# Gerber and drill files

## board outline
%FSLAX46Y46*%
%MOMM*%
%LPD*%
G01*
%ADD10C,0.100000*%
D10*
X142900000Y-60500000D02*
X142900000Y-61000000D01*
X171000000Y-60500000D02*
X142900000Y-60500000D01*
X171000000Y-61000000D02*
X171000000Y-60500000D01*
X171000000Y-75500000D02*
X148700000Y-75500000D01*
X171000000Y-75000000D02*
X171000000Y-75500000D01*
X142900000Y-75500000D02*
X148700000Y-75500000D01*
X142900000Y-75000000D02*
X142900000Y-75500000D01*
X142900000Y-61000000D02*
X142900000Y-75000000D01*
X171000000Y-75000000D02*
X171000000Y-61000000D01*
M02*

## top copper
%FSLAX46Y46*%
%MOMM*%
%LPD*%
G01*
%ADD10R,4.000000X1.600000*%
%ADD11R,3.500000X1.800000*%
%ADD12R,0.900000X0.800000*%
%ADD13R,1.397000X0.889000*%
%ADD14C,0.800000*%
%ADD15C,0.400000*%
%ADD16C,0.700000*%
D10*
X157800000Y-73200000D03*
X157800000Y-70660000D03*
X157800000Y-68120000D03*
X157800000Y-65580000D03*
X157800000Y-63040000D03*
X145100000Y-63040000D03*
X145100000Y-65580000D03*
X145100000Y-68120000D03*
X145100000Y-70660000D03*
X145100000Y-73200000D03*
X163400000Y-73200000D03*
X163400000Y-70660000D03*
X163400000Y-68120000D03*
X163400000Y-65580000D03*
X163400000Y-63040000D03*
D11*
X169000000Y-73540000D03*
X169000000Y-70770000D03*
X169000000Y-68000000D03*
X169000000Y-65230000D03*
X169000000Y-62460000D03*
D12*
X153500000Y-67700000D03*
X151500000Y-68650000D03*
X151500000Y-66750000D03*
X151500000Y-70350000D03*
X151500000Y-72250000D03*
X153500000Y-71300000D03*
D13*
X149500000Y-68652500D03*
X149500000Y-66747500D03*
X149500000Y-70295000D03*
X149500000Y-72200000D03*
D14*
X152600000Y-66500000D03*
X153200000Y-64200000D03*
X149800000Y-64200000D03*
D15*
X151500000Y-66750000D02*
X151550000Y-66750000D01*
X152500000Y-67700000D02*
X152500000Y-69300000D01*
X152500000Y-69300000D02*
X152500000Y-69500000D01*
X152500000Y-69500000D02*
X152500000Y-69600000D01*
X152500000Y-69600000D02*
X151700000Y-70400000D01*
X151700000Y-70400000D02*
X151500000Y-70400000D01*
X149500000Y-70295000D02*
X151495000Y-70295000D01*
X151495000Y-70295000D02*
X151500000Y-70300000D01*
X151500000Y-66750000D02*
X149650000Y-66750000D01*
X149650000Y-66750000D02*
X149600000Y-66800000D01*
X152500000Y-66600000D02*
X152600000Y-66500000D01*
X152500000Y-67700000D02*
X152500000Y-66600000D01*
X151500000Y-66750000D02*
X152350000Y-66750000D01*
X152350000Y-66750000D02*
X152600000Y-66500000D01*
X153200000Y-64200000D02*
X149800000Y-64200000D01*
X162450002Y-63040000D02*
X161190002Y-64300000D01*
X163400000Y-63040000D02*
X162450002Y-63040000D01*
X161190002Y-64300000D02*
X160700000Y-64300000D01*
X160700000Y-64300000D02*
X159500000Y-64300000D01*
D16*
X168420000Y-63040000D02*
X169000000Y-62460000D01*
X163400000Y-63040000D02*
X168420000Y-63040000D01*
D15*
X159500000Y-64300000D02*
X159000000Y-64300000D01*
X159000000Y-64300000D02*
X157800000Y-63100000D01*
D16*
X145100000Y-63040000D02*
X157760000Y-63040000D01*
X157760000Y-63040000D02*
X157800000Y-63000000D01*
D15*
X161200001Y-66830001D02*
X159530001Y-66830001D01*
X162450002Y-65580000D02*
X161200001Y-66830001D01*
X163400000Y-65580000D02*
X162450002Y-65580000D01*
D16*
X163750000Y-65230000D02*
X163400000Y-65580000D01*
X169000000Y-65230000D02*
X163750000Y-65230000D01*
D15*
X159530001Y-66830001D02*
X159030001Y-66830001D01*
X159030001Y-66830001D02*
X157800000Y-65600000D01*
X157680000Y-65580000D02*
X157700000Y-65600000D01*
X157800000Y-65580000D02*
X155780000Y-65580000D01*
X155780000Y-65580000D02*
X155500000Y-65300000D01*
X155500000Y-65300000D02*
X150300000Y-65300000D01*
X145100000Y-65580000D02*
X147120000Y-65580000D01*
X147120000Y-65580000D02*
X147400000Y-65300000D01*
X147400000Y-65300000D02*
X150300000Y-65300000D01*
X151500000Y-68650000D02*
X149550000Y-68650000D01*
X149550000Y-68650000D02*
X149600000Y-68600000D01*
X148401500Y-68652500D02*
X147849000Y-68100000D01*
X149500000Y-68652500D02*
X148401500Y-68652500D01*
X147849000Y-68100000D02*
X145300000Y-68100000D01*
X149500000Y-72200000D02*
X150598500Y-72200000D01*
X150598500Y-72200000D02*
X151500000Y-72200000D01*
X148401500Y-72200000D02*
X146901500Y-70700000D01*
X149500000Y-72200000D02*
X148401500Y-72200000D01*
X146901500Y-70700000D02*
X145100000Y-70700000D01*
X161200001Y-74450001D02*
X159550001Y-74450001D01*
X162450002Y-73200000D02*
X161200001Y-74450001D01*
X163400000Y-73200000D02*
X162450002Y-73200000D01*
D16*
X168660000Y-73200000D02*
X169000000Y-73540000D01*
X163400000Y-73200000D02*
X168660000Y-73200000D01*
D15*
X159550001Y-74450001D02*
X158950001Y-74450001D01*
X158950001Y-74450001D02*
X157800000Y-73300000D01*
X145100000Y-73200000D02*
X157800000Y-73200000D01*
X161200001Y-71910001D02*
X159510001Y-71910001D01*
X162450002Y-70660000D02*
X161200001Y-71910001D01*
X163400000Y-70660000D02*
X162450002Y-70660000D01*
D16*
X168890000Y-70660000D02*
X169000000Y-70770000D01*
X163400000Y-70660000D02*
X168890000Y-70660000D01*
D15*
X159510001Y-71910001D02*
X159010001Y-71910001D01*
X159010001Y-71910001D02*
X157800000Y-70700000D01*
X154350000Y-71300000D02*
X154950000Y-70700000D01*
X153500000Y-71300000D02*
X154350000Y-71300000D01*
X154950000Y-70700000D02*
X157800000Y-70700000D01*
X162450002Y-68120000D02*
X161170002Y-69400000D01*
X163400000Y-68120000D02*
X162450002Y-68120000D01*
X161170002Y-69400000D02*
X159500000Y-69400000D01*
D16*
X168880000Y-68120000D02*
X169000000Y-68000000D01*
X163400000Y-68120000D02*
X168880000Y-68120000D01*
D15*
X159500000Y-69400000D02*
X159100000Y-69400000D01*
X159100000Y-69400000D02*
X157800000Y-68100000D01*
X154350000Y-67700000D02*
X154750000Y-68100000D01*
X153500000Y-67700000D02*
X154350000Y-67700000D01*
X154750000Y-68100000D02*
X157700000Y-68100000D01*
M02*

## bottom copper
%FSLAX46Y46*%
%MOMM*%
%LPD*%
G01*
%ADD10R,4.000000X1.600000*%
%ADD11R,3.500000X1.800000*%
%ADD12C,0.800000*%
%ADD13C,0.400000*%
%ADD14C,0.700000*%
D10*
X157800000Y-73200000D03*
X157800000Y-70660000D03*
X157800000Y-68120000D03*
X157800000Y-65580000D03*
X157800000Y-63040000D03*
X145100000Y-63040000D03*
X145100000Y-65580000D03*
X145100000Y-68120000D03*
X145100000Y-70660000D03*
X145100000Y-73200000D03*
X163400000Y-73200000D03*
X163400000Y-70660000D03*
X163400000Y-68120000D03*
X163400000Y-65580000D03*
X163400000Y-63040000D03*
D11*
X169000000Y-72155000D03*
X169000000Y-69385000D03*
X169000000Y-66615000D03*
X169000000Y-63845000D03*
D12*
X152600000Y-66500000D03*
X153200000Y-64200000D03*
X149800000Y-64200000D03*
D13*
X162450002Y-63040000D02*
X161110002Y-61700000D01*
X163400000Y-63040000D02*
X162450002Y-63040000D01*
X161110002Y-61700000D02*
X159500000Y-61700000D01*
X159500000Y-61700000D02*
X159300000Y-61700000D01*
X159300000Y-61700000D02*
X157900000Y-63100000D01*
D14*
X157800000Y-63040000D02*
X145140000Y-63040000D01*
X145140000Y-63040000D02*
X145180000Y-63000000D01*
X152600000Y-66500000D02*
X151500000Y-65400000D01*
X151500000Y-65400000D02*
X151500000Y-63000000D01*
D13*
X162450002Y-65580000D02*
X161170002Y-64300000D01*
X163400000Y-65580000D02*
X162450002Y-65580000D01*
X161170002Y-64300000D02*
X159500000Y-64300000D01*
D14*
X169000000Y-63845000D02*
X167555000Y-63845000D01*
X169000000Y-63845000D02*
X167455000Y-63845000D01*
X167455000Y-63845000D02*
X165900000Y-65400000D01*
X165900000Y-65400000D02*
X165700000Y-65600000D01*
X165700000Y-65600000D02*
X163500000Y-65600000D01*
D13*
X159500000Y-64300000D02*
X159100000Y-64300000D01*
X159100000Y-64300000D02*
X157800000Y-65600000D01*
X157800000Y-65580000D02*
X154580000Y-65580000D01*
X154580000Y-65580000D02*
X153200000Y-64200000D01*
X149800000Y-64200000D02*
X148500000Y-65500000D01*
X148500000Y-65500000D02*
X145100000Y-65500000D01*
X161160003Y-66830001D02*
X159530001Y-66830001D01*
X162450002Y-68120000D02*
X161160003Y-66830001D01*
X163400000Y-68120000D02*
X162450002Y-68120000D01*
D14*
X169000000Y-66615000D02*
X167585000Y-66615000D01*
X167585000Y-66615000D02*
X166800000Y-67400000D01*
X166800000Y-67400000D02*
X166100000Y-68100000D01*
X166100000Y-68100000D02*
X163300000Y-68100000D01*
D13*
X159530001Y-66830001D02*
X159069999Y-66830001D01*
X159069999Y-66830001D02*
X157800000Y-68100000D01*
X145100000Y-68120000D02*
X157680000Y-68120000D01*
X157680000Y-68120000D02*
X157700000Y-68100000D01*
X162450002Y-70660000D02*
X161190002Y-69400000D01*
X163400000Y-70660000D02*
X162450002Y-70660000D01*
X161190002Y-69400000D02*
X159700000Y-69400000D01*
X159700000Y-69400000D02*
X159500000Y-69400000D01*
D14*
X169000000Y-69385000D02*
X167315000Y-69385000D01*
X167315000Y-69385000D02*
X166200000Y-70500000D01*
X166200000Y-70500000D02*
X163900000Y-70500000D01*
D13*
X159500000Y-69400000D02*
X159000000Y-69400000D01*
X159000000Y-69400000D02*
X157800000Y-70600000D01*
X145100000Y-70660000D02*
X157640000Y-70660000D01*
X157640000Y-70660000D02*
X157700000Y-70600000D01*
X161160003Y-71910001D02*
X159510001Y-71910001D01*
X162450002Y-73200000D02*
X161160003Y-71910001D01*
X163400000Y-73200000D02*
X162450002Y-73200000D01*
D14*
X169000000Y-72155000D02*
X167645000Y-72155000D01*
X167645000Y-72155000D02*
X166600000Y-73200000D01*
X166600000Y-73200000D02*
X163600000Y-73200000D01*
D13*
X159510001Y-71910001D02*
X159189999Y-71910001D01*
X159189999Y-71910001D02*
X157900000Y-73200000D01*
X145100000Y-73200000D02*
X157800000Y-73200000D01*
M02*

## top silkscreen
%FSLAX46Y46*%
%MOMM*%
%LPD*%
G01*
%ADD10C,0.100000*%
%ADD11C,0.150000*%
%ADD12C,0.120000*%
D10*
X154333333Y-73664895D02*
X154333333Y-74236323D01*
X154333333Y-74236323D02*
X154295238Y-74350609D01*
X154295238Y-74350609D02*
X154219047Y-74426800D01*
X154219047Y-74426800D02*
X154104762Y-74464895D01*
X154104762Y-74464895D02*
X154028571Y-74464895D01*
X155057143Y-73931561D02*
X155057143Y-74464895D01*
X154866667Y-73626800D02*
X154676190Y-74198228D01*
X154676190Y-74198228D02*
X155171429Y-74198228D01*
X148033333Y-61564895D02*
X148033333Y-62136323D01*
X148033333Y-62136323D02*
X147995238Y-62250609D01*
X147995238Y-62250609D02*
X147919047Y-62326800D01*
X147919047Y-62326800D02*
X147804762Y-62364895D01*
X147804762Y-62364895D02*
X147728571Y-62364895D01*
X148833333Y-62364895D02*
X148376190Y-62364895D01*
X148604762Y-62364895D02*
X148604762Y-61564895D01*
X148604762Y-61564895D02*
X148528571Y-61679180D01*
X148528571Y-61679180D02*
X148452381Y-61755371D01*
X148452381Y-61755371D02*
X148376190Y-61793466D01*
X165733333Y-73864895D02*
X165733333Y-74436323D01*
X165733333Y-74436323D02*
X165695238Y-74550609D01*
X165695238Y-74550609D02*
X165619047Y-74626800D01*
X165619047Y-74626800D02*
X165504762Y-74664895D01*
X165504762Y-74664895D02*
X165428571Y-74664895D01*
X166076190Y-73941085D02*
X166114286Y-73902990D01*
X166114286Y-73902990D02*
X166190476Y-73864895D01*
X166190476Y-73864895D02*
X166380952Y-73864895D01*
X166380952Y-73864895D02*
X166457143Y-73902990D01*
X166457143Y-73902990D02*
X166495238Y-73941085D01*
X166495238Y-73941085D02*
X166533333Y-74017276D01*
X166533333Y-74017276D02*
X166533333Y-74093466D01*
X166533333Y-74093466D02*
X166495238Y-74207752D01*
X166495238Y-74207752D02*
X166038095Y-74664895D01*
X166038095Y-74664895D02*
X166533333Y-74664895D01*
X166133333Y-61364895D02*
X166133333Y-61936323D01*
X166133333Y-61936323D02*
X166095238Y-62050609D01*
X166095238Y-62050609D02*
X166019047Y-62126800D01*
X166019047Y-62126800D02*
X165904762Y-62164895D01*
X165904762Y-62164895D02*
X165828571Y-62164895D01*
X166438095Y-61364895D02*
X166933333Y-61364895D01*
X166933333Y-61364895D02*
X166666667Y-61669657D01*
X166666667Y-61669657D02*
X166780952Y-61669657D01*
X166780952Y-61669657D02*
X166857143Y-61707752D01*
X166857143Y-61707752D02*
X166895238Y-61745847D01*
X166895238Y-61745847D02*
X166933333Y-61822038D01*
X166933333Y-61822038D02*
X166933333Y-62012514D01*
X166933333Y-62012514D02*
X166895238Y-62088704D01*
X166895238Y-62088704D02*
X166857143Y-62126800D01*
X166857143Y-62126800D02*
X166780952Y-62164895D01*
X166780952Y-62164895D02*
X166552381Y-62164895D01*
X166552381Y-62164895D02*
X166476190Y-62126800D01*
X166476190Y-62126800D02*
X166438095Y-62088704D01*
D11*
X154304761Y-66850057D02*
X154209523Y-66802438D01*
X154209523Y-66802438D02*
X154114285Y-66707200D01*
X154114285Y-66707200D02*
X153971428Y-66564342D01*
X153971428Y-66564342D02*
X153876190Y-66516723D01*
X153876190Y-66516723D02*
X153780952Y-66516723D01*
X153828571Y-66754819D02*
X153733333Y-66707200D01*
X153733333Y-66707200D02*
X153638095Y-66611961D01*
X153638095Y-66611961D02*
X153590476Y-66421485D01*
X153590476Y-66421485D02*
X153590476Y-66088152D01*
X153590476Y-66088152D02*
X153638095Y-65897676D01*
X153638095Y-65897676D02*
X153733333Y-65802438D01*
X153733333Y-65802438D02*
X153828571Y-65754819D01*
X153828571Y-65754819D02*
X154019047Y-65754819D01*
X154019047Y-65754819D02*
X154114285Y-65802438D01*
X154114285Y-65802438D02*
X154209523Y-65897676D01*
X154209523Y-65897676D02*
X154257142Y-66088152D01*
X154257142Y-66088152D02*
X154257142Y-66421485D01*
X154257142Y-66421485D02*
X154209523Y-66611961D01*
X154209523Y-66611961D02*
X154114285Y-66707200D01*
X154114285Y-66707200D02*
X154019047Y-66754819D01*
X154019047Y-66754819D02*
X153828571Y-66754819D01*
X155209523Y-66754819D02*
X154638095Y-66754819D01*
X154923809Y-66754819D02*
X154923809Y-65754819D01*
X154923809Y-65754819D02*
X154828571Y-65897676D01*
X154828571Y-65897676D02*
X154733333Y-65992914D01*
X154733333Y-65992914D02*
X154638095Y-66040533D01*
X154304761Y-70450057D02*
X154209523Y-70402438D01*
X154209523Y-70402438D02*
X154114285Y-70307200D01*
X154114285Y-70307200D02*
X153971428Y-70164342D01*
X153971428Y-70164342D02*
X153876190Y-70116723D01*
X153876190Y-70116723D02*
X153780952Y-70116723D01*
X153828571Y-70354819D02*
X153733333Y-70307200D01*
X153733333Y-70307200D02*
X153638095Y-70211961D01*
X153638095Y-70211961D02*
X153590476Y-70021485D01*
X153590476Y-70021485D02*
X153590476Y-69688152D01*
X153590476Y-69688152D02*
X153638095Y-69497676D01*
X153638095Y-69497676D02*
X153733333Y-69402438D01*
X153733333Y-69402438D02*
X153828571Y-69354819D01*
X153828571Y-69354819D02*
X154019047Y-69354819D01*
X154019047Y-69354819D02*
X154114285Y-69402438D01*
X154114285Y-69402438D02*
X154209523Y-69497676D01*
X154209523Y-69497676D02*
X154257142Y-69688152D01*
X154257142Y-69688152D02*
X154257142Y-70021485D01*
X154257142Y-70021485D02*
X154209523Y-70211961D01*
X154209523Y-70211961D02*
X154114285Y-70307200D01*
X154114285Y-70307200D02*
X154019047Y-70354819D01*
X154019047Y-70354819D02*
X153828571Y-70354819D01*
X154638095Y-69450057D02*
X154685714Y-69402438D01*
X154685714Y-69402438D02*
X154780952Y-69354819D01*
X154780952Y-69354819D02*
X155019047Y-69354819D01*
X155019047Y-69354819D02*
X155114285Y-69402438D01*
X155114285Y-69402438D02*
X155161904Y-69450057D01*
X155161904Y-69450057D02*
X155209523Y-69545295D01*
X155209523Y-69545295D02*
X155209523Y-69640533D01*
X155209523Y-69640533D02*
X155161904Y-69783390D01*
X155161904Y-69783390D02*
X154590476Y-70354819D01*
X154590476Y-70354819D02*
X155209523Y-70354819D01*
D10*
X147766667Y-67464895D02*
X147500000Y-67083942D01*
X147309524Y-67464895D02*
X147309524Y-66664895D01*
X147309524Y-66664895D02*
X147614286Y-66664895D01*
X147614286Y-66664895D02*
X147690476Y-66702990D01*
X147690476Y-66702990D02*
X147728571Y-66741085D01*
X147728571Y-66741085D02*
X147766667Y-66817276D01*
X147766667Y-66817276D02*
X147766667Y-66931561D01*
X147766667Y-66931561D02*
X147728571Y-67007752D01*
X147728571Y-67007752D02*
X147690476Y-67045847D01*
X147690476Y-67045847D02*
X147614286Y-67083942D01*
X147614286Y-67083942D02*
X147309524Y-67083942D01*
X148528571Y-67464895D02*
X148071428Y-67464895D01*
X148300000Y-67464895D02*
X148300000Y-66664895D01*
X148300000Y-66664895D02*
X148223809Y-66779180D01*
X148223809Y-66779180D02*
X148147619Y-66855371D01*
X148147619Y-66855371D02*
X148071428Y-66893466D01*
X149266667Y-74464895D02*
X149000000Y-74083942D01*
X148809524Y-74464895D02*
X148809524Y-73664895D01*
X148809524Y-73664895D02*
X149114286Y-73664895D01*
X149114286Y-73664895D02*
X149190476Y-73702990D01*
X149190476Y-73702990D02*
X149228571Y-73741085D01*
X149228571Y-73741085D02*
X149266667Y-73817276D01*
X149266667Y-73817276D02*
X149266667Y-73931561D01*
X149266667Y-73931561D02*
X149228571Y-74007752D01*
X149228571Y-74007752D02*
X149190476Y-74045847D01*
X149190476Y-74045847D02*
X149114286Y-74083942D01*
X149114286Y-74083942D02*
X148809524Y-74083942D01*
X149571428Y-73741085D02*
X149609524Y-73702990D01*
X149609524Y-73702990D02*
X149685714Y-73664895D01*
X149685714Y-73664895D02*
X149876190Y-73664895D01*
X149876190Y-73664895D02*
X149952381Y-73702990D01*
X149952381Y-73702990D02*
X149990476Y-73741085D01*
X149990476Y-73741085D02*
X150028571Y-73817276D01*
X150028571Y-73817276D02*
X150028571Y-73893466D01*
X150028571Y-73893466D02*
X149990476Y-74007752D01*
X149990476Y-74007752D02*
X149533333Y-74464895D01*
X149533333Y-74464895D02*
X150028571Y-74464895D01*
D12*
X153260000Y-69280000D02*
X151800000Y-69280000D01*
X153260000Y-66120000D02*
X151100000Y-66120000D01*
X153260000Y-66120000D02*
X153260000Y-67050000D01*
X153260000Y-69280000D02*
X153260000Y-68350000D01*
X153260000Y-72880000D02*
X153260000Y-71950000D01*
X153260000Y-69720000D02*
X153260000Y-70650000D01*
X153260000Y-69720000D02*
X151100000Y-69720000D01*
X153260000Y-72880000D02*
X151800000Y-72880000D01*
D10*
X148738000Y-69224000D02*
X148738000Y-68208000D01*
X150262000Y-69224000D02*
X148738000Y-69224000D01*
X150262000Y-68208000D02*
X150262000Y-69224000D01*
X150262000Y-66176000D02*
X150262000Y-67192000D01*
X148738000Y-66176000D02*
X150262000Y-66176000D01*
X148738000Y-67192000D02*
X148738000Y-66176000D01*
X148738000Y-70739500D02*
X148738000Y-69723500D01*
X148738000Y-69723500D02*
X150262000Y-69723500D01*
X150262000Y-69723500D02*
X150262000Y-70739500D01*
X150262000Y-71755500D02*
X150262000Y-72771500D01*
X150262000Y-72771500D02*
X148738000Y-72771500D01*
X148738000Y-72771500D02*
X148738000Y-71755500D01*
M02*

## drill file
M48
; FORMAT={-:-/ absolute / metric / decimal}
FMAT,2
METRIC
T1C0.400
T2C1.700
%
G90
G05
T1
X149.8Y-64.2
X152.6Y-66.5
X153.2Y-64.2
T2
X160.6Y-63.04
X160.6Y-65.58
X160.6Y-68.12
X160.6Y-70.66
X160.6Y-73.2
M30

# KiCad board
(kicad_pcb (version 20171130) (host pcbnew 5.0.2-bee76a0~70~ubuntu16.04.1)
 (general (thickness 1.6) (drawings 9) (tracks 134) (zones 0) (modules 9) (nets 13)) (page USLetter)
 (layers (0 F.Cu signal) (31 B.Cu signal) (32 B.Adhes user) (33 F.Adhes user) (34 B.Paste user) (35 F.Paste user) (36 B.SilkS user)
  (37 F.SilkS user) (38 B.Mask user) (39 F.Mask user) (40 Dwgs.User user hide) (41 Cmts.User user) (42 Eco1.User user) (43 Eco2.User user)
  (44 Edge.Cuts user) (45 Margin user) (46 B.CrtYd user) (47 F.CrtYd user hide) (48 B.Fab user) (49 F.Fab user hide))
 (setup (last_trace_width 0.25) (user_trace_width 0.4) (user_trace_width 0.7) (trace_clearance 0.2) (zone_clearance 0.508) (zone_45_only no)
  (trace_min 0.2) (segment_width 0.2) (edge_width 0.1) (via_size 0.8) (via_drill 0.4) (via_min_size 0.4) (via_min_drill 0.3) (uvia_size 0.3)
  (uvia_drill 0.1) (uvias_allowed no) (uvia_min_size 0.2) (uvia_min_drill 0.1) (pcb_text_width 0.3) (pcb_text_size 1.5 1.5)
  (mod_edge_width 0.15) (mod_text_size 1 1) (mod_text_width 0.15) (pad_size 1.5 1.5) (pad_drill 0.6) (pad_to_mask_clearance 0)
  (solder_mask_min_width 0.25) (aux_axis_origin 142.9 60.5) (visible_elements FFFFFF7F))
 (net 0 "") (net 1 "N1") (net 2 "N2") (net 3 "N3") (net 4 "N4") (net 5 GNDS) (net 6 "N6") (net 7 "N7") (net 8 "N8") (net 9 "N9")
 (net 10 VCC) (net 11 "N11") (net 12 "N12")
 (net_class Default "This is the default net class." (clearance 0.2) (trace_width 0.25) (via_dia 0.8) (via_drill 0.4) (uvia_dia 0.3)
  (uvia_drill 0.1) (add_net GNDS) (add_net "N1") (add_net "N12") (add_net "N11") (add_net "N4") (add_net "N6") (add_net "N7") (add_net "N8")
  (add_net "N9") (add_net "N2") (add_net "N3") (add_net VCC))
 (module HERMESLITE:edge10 (layer F.Cu) (at 157.8 73.2 270)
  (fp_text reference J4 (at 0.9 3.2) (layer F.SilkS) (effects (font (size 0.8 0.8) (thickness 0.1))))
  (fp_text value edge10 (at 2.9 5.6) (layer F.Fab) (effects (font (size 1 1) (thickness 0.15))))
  (pad 1 smd rect (at 0 0 270) (size 1.6 4) (layers F.Cu F.Paste F.Mask) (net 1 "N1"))
  (pad 2 smd rect (at -2.54 0 270) (size 1.6 4) (layers F.Cu F.Paste F.Mask) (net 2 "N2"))
  (pad 3 smd rect (at -5.08 0 270) (size 1.6 4) (layers F.Cu F.Paste F.Mask) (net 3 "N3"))
  (pad 4 smd rect (at -7.62 0 270) (size 1.6 4) (layers F.Cu F.Paste F.Mask) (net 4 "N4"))
  (pad 5 smd rect (at -10.16 0 270) (size 1.6 4) (layers F.Cu F.Paste F.Mask) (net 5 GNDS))
  (pad 6 smd rect (at 0 0 270) (size 1.6 4) (layers B.Cu B.Paste B.Mask) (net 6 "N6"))
  (pad 7 smd rect (at -2.54 0 270) (size 1.6 4) (layers B.Cu B.Paste B.Mask) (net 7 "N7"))
  (pad 8 smd rect (at -5.08 0 270) (size 1.6 4) (layers B.Cu B.Paste B.Mask) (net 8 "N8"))
  (pad 9 smd rect (at -7.62 0 270) (size 1.6 4) (layers B.Cu B.Paste B.Mask) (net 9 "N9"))
  (pad 10 smd rect (at -10.16 0 270) (size 1.6 4) (layers B.Cu B.Paste B.Mask) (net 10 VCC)))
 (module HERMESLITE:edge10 (layer F.Cu) (at 145.1 73.2 270)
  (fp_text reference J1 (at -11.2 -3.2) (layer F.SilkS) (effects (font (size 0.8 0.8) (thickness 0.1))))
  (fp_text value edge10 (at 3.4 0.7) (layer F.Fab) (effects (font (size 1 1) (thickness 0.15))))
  (pad 10 smd rect (at -10.16 0 270) (size 1.6 4) (layers B.Cu B.Paste B.Mask) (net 10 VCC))
  (pad 9 smd rect (at -7.62 0 270) (size 1.6 4) (layers B.Cu B.Paste B.Mask) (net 9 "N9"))
  (pad 8 smd rect (at -5.08 0 270) (size 1.6 4) (layers B.Cu B.Paste B.Mask) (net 8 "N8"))
  (pad 7 smd rect (at -2.54 0 270) (size 1.6 4) (layers B.Cu B.Paste B.Mask) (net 7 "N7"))
  (pad 6 smd rect (at 0 0 270) (size 1.6 4) (layers B.Cu B.Paste B.Mask) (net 6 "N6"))
  (pad 5 smd rect (at -10.16 0 270) (size 1.6 4) (layers F.Cu F.Paste F.Mask) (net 5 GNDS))
  (pad 4 smd rect (at -7.62 0 270) (size 1.6 4) (layers F.Cu F.Paste F.Mask) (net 4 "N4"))
  (pad 3 smd rect (at -5.08 0 270) (size 1.6 4) (layers F.Cu F.Paste F.Mask) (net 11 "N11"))
  (pad 2 smd rect (at -2.54 0 270) (size 1.6 4) (layers F.Cu F.Paste F.Mask) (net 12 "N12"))
  (pad 1 smd rect (at 0 0 270) (size 1.6 4) (layers F.Cu F.Paste F.Mask) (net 1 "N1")))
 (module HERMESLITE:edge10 (layer F.Cu) (at 163.4 73.2 270)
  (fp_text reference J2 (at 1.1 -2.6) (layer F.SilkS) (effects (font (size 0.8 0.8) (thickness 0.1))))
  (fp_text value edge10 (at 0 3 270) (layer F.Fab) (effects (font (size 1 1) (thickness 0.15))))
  (pad 1 smd rect (at 0 0 270) (size 1.6 4) (layers F.Cu F.Paste F.Mask) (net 1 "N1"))
  (pad 2 smd rect (at -2.54 0 270) (size 1.6 4) (layers F.Cu F.Paste F.Mask) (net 2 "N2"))
  (pad 3 smd rect (at -5.08 0 270) (size 1.6 4) (layers F.Cu F.Paste F.Mask) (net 3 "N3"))
  (pad 4 smd rect (at -7.62 0 270) (size 1.6 4) (layers F.Cu F.Paste F.Mask) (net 4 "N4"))
  (pad 5 smd rect (at -10.16 0 270) (size 1.6 4) (layers F.Cu F.Paste F.Mask) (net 5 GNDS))
  (pad 6 smd rect (at 0 0 270) (size 1.6 4) (layers B.Cu B.Paste B.Mask) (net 6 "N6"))
  (pad 7 smd rect (at -2.54 0 270) (size 1.6 4) (layers B.Cu B.Paste B.Mask) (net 7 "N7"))
  (pad 8 smd rect (at -5.08 0 270) (size 1.6 4) (layers B.Cu B.Paste B.Mask) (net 8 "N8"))
  (pad 9 smd rect (at -7.62 0 270) (size 1.6 4) (layers B.Cu B.Paste B.Mask) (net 9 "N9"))
  (pad 10 smd rect (at -10.16 0 270) (size 1.6 4) (layers B.Cu B.Paste B.Mask) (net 10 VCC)))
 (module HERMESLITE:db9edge (layer F.Cu) (at 169 73.54 270)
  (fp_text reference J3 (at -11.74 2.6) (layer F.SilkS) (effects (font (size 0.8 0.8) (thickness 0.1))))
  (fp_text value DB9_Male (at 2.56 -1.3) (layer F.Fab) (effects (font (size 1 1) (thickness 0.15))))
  (pad 1 smd rect (at 0 0 270) (size 1.8 3.5) (layers F.Cu F.Paste F.Mask) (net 1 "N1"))
  (pad 2 smd rect (at -2.77 0 270) (size 1.8 3.5) (layers F.Cu F.Paste F.Mask) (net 2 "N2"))
  (pad 3 smd rect (at -5.54 0 270) (size 1.8 3.5) (layers F.Cu F.Paste F.Mask) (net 3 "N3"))
  (pad 4 smd rect (at -8.31 0 270) (size 1.8 3.5) (layers F.Cu F.Paste F.Mask) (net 4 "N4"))
  (pad 5 smd rect (at -11.08 0 270) (size 1.8 3.5) (layers F.Cu F.Paste F.Mask) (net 5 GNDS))
  (pad 6 smd rect (at -1.385 0 270) (size 1.8 3.5) (layers B.Cu B.Paste B.Mask) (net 6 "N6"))
  (pad 7 smd rect (at -4.155 0 270) (size 1.8 3.5) (layers B.Cu B.Paste B.Mask) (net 7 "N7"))
  (pad 8 smd rect (at -6.925 0 270) (size 1.8 3.5) (layers B.Cu B.Paste B.Mask) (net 8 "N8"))
  (pad 9 smd rect (at -9.695 0 270) (size 1.8 3.5) (layers B.Cu B.Paste B.Mask) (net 9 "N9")))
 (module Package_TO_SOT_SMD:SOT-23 (layer F.Cu) (at 152.5 67.7)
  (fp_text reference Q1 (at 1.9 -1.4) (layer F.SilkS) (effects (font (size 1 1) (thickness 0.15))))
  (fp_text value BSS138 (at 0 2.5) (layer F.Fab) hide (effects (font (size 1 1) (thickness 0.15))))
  (fp_line (start 0.76 1.58) (end -0.7 1.58) (layer F.SilkS) (width 0.12))
  (fp_line (start 0.76 -1.58) (end -1.4 -1.58) (layer F.SilkS) (width 0.12))
  (fp_line (start 0.76 -1.58) (end 0.76 -0.65) (layer F.SilkS) (width 0.12))
  (fp_line (start 0.76 1.58) (end 0.76 0.65) (layer F.SilkS) (width 0.12))
  (pad 3 smd rect (at 1 0) (size 0.9 0.8) (layers F.Cu F.Paste F.Mask) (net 3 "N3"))
  (pad 2 smd rect (at -1 0.95) (size 0.9 0.8) (layers F.Cu F.Paste F.Mask) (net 11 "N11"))
  (pad 1 smd rect (at -1 -0.95) (size 0.9 0.8) (layers F.Cu F.Paste F.Mask) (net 10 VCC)))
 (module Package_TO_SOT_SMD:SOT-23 (layer F.Cu) (at 152.5 71.3)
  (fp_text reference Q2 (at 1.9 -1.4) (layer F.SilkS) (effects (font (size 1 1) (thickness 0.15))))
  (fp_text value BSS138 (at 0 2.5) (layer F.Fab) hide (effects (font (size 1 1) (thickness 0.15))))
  (fp_line (start 0.76 1.58) (end 0.76 0.65) (layer F.SilkS) (width 0.12))
  (fp_line (start 0.76 -1.58) (end 0.76 -0.65) (layer F.SilkS) (width 0.12))
  (fp_line (start 0.76 -1.58) (end -1.4 -1.58) (layer F.SilkS) (width 0.12))
  (fp_line (start 0.76 1.58) (end -0.7 1.58) (layer F.SilkS) (width 0.12))
  (pad 1 smd rect (at -1 -0.95) (size 0.9 0.8) (layers F.Cu F.Paste F.Mask) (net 10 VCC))
  (pad 2 smd rect (at -1 0.95) (size 0.9 0.8) (layers F.Cu F.Paste F.Mask) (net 12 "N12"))
  (pad 3 smd rect (at 1 0) (size 0.9 0.8) (layers F.Cu F.Paste F.Mask) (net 2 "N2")))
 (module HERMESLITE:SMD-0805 (layer F.Cu) (at 149.5 67.7 270)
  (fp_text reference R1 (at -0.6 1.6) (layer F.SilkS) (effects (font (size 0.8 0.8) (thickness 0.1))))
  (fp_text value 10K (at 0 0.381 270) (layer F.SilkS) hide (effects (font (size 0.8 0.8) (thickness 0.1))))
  (fp_line (start 1.524 0.762) (end 0.508 0.762) (layer F.SilkS) (width 0.1))
  (fp_line (start 1.524 -0.762) (end 1.524 0.762) (layer F.SilkS) (width 0.1))
  (fp_line (start 0.508 -0.762) (end 1.524 -0.762) (layer F.SilkS) (width 0.1))
  (fp_line (start -1.524 -0.762) (end -0.508 -0.762) (layer F.SilkS) (width 0.1))
  (fp_line (start -1.524 0.762) (end -1.524 -0.762) (layer F.SilkS) (width 0.1))
  (fp_line (start -0.508 0.762) (end -1.524 0.762) (layer F.SilkS) (width 0.1))
  (pad 2 smd rect (at 0.9525 0 270) (size 0.889 1.397) (layers F.Cu F.Paste F.Mask) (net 11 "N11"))
  (pad 1 smd rect (at -0.9525 0 270) (size 0.889 1.397) (layers F.Cu F.Paste F.Mask) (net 10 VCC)))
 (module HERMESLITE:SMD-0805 (layer F.Cu) (at 149.5 71.2475 270)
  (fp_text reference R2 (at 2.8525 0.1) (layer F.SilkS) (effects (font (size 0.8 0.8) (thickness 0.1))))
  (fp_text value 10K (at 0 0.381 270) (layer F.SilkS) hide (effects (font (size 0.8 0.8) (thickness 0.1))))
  (fp_line (start -0.508 0.762) (end -1.524 0.762) (layer F.SilkS) (width 0.1))
  (fp_line (start -1.524 0.762) (end -1.524 -0.762) (layer F.SilkS) (width 0.1))
  (fp_line (start -1.524 -0.762) (end -0.508 -0.762) (layer F.SilkS) (width 0.1))
  (fp_line (start 0.508 -0.762) (end 1.524 -0.762) (layer F.SilkS) (width 0.1))
  (fp_line (start 1.524 -0.762) (end 1.524 0.762) (layer F.SilkS) (width 0.1))
  (fp_line (start 1.524 0.762) (end 0.508 0.762) (layer F.SilkS) (width 0.1))
  (pad 1 smd rect (at -0.9525 0 270) (size 0.889 1.397) (layers F.Cu F.Paste F.Mask) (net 10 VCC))
  (pad 2 smd rect (at 0.9525 0 270) (size 0.889 1.397) (layers F.Cu F.Paste F.Mask) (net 12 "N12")))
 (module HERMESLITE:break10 (layer F.Cu) (at 160.6 73.2)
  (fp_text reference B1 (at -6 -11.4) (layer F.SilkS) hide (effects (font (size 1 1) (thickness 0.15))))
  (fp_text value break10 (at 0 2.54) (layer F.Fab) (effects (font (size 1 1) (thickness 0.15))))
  (pad "" np_thru_hole circle (at 0 -10.16) (size 1.7 1.7) (drill 1.7) (layers *.Cu *.Mask))
  (pad "" np_thru_hole circle (at 0 -7.62) (size 1.7 1.7) (drill 1.7) (layers *.Cu *.Mask))
  (pad "" np_thru_hole circle (at 0 -5.08) (size 1.7 1.7) (drill 1.7) (layers *.Cu *.Mask))
  (pad "" np_thru_hole circle (at 0 -2.54) (size 1.7 1.7) (drill 1.7) (layers *.Cu *.Mask))
  (pad "" np_thru_hole circle (at 0 0) (size 1.7 1.7) (drill 1.7) (layers *.Cu *.Mask)))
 (gr_line (start 142.9 60.5) (end 142.9 61) (layer Edge.Cuts) (width 0.1))
 (gr_line (start 171 60.5) (end 142.9 60.5) (layer Edge.Cuts) (width 0.1))
 (gr_line (start 171 61) (end 171 60.5) (layer Edge.Cuts) (width 0.1))
 (gr_line (start 171 75.5) (end 148.7 75.5) (layer Edge.Cuts) (width 0.1))
 (gr_line (start 171 75) (end 171 75.5) (layer Edge.Cuts) (width 0.1))
 (gr_line (start 142.9 75.5) (end 148.7 75.5) (layer Edge.Cuts) (width 0.1))
 (gr_line (start 142.9 75) (end 142.9 75.5) (layer Edge.Cuts) (width 0.1))
 (gr_line (start 142.9 61) (end 142.9 75) (layer Edge.Cuts) (width 0.1))
 (gr_line (start 171 75) (end 171 61) (layer Edge.Cuts) (width 0.1))
 (segment (start 162.450002 63.04) (end 161.110002 61.7) (width 0.4) (layer B.Cu) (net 10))
 (segment (start 163.4 63.04) (end 162.450002 63.04) (width 0.4) (layer B.Cu) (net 10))
 (segment (start 161.110002 61.7) (end 159.5 61.7) (width 0.4) (layer B.Cu) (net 10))
 (segment (start 159.5 61.7) (end 159.3 61.7) (width 0.4) (layer B.Cu) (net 10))
 (segment (start 159.3 61.7) (end 157.9 63.1) (width 0.4) (layer B.Cu) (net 10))
 (segment (start 151.5 66.75) (end 151.55 66.75) (width 0.4) (layer F.Cu) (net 10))
 (segment (start 152.5 67.7) (end 152.5 69.3) (width 0.4) (layer F.Cu) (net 10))
 (segment (start 152.5 69.3) (end 152.5 69.5) (width 0.4) (layer F.Cu) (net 10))
 (segment (start 152.5 69.5) (end 152.5 69.6) (width 0.4) (layer F.Cu) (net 10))
 (segment (start 152.5 69.6) (end 151.7 70.4) (width 0.4) (layer F.Cu) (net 10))
 (segment (start 151.7 70.4) (end 151.5 70.4) (width 0.4) (layer F.Cu) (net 10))
 (segment (start 149.5 70.295) (end 151.495 70.295) (width 0.4) (layer F.Cu) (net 10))
 (segment (start 151.495 70.295) (end 151.5 70.3) (width 0.4) (layer F.Cu) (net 10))
 (segment (start 151.5 66.75) (end 149.65 66.75) (width 0.4) (layer F.Cu) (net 10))
 (segment (start 149.65 66.75) (end 149.6 66.8) (width 0.4) (layer F.Cu) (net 10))
 (segment (start 157.8 63.04) (end 145.14 63.04) (width 0.7) (layer B.Cu) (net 10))
 (segment (start 145.14 63.04) (end 145.18 63) (width 0.7) (layer B.Cu) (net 10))
 (via (at 152.6 66.5) (size 0.8) (drill 0.4) (layers F.Cu B.Cu) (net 10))
 (segment (start 152.5 66.6) (end 152.6 66.5) (width 0.4) (layer F.Cu) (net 10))
 (segment (start 152.5 67.7) (end 152.5 66.6) (width 0.4) (layer F.Cu) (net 10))
 (segment (start 151.5 66.75) (end 152.35 66.75) (width 0.4) (layer F.Cu) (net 10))
 (segment (start 152.35 66.75) (end 152.6 66.5) (width 0.4) (layer F.Cu) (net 10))
 (segment (start 152.6 66.5) (end 151.5 65.4) (width 0.7) (layer B.Cu) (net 10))
 (segment (start 151.5 65.4) (end 151.5 63) (width 0.7) (layer B.Cu) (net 10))
 (segment (start 162.450002 65.58) (end 161.170002 64.3) (width 0.4) (layer B.Cu) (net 9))
 (segment (start 163.4 65.58) (end 162.450002 65.58) (width 0.4) (layer B.Cu) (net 9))
 (segment (start 161.170002 64.3) (end 159.5 64.3) (width 0.4) (layer B.Cu) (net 9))
 (segment (start 169 63.845) (end 167.555 63.845) (width 0.7) (layer B.Cu) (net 9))
 (segment (start 169 63.845) (end 167.455 63.845) (width 0.7) (layer B.Cu) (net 9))
 (segment (start 167.455 63.845) (end 165.9 65.4) (width 0.7) (layer B.Cu) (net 9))
 (segment (start 165.9 65.4) (end 165.7 65.6) (width 0.7) (layer B.Cu) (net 9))
 (segment (start 165.7 65.6) (end 163.5 65.6) (width 0.7) (layer B.Cu) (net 9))
 (segment (start 159.5 64.3) (end 159.1 64.3) (width 0.4) (layer B.Cu) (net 9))
 (segment (start 159.1 64.3) (end 157.8 65.6) (width 0.4) (layer B.Cu) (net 9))
 (via (at 153.2 64.2) (size 0.8) (drill 0.4) (layers F.Cu B.Cu) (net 9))
 (segment (start 157.8 65.58) (end 154.58 65.58) (width 0.4) (layer B.Cu) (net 9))
 (segment (start 154.58 65.58) (end 153.2 64.2) (width 0.4) (layer B.Cu) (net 9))
 (via (at 149.8 64.2) (size 0.8) (drill 0.4) (layers F.Cu B.Cu) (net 9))
 (segment (start 153.2 64.2) (end 149.8 64.2) (width 0.4) (layer F.Cu) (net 9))
 (segment (start 149.8 64.2) (end 148.5 65.5) (width 0.4) (layer B.Cu) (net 9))
 (segment (start 148.5 65.5) (end 145.1 65.5) (width 0.4) (layer B.Cu) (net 9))
 (segment (start 161.160003 66.830001) (end 159.530001 66.830001) (width 0.4) (layer B.Cu) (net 8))
 (segment (start 162.450002 68.12) (end 161.160003 66.830001) (width 0.4) (layer B.Cu) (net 8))
 (segment (start 163.4 68.12) (end 162.450002 68.12) (width 0.4) (layer B.Cu) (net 8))
 (segment (start 169 66.615) (end 167.585 66.615) (width 0.7) (layer B.Cu) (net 8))
 (segment (start 167.585 66.615) (end 166.8 67.4) (width 0.7) (layer B.Cu) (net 8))
 (segment (start 166.8 67.4) (end 166.1 68.1) (width 0.7) (layer B.Cu) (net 8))
 (segment (start 166.1 68.1) (end 163.3 68.1) (width 0.7) (layer B.Cu) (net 8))
 (segment (start 159.530001 66.830001) (end 159.069999 66.830001) (width 0.4) (layer B.Cu) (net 8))
 (segment (start 159.069999 66.830001) (end 157.8 68.1) (width 0.4) (layer B.Cu) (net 8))
 (segment (start 145.1 68.12) (end 157.68 68.12) (width 0.4) (layer B.Cu) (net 8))
 (segment (start 157.68 68.12) (end 157.7 68.1) (width 0.4) (layer B.Cu) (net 8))
 (segment (start 162.450002 70.66) (end 161.190002 69.4) (width 0.4) (layer B.Cu) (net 7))
 (segment (start 163.4 70.66) (end 162.450002 70.66) (width 0.4) (layer B.Cu) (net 7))
 (segment (start 161.190002 69.4) (end 159.7 69.4) (width 0.4) (layer B.Cu) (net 7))
 (segment (start 159.7 69.4) (end 159.5 69.4) (width 0.4) (layer B.Cu) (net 7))
 (segment (start 169 69.385) (end 167.315 69.385) (width 0.7) (layer B.Cu) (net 7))
 (segment (start 167.315 69.385) (end 166.2 70.5) (width 0.7) (layer B.Cu) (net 7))
 (segment (start 166.2 70.5) (end 163.9 70.5) (width 0.7) (layer B.Cu) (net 7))
 (segment (start 159.5 69.4) (end 159 69.4) (width 0.4) (layer B.Cu) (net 7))
 (segment (start 159 69.4) (end 157.8 70.6) (width 0.4) (layer B.Cu) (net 7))
 (segment (start 145.1 70.66) (end 157.64 70.66) (width 0.4) (layer B.Cu) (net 7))
 (segment (start 157.64 70.66) (end 157.7 70.6) (width 0.4) (layer B.Cu) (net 7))
 (segment (start 161.160003 71.910001) (end 159.510001 71.910001) (width 0.4) (layer B.Cu) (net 6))
 (segment (start 162.450002 73.2) (end 161.160003 71.910001) (width 0.4) (layer B.Cu) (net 6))
 (segment (start 163.4 73.2) (end 162.450002 73.2) (width 0.4) (layer B.Cu) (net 6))
 (segment (start 169 72.155) (end 167.645 72.155) (width 0.7) (layer B.Cu) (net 6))
 (segment (start 167.645 72.155) (end 166.6 73.2) (width 0.7) (layer B.Cu) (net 6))
 (segment (start 166.6 73.2) (end 163.6 73.2) (width 0.7) (layer B.Cu) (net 6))
 (segment (start 159.510001 71.910001) (end 159.189999 71.910001) (width 0.4) (layer B.Cu) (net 6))
 (segment (start 159.189999 71.910001) (end 157.9 73.2) (width 0.4) (layer B.Cu) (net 6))
 (segment (start 145.1 73.2) (end 157.8 73.2) (width 0.4) (layer B.Cu) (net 6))
 (segment (start 162.450002 63.04) (end 161.190002 64.3) (width 0.4) (layer F.Cu) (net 5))
 (segment (start 163.4 63.04) (end 162.450002 63.04) (width 0.4) (layer F.Cu) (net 5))
 (segment (start 161.190002 64.3) (end 160.7 64.3) (width 0.4) (layer F.Cu) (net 5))
 (segment (start 160.7 64.3) (end 159.5 64.3) (width 0.4) (layer F.Cu) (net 5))
 (segment (start 168.42 63.04) (end 169 62.46) (width 0.7) (layer F.Cu) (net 5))
 (segment (start 163.4 63.04) (end 168.42 63.04) (width 0.7) (layer F.Cu) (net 5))
 (segment (start 159.5 64.3) (end 159 64.3) (width 0.4) (layer F.Cu) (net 5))
 (segment (start 159 64.3) (end 157.8 63.1) (width 0.4) (layer F.Cu) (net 5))
 (segment (start 145.1 63.04) (end 157.76 63.04) (width 0.7) (layer F.Cu) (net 5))
 (segment (start 157.76 63.04) (end 157.8 63) (width 0.7) (layer F.Cu) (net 5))
 (segment (start 161.200001 66.830001) (end 159.530001 66.830001) (width 0.4) (layer F.Cu) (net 4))
 (segment (start 162.450002 65.58) (end 161.200001 66.830001) (width 0.4) (layer F.Cu) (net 4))
 (segment (start 163.4 65.58) (end 162.450002 65.58) (width 0.4) (layer F.Cu) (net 4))
 (segment (start 163.75 65.23) (end 163.4 65.58) (width 0.7) (layer F.Cu) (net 4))
 (segment (start 169 65.23) (end 163.75 65.23) (width 0.7) (layer F.Cu) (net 4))
 (segment (start 159.530001 66.830001) (end 159.030001 66.830001) (width 0.4) (layer F.Cu) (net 4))
 (segment (start 159.030001 66.830001) (end 157.8 65.6) (width 0.4) (layer F.Cu) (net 4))
 (segment (start 157.68 65.58) (end 157.7 65.6) (width 0.4) (layer F.Cu) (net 4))
 (segment (start 157.8 65.58) (end 155.78 65.58) (width 0.4) (layer F.Cu) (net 4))
 (segment (start 155.78 65.58) (end 155.5 65.3) (width 0.4) (layer F.Cu) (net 4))
 (segment (start 155.5 65.3) (end 150.3 65.3) (width 0.4) (layer F.Cu) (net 4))
 (segment (start 145.1 65.58) (end 147.12 65.58) (width 0.4) (layer F.Cu) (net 4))
 (segment (start 147.12 65.58) (end 147.4 65.3) (width 0.4) (layer F.Cu) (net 4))
 (segment (start 147.4 65.3) (end 150.3 65.3) (width 0.4) (layer F.Cu) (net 4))
 (segment (start 151.5 68.65) (end 149.55 68.65) (width 0.4) (layer F.Cu) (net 11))
 (segment (start 149.55 68.65) (end 149.6 68.6) (width 0.4) (layer F.Cu) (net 11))
 (segment (start 148.4015 68.6525) (end 147.849 68.1) (width 0.4) (layer F.Cu) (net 11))
 (segment (start 149.5 68.6525) (end 148.4015 68.6525) (width 0.4) (layer F.Cu) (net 11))
 (segment (start 147.849 68.1) (end 145.3 68.1) (width 0.4) (layer F.Cu) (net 11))
 (segment (start 149.5 72.2) (end 150.5985 72.2) (width 0.4) (layer F.Cu) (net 12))
 (segment (start 150.5985 72.2) (end 151.5 72.2) (width 0.4) (layer F.Cu) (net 12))
 (segment (start 148.4015 72.2) (end 146.9015 70.7) (width 0.4) (layer F.Cu) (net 12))
 (segment (start 149.5 72.2) (end 148.4015 72.2) (width 0.4) (layer F.Cu) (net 12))
 (segment (start 146.9015 70.7) (end 145.1 70.7) (width 0.4) (layer F.Cu) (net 12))
 (segment (start 161.200001 74.450001) (end 159.550001 74.450001) (width 0.4) (layer F.Cu) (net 1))
 (segment (start 162.450002 73.2) (end 161.200001 74.450001) (width 0.4) (layer F.Cu) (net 1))
 (segment (start 163.4 73.2) (end 162.450002 73.2) (width 0.4) (layer F.Cu) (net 1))
 (segment (start 168.66 73.2) (end 169 73.54) (width 0.7) (layer F.Cu) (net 1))
 (segment (start 163.4 73.2) (end 168.66 73.2) (width 0.7) (layer F.Cu) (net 1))
 (segment (start 159.550001 74.450001) (end 158.950001 74.450001) (width 0.4) (layer F.Cu) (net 1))
 (segment (start 158.950001 74.450001) (end 157.8 73.3) (width 0.4) (layer F.Cu) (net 1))
 (segment (start 145.1 73.2) (end 157.8 73.2) (width 0.4) (layer F.Cu) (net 1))
 (segment (start 161.200001 71.910001) (end 159.510001 71.910001) (width 0.4) (layer F.Cu) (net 2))
 (segment (start 162.450002 70.66) (end 161.200001 71.910001) (width 0.4) (layer F.Cu) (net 2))
 (segment (start 163.4 70.66) (end 162.450002 70.66) (width 0.4) (layer F.Cu) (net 2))
 (segment (start 168.89 70.66) (end 169 70.77) (width 0.7) (layer F.Cu) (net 2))
 (segment (start 163.4 70.66) (end 168.89 70.66) (width 0.7) (layer F.Cu) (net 2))
 (segment (start 159.510001 71.910001) (end 159.010001 71.910001) (width 0.4) (layer F.Cu) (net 2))
 (segment (start 159.010001 71.910001) (end 157.8 70.7) (width 0.4) (layer F.Cu) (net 2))
 (segment (start 154.35 71.3) (end 154.95 70.7) (width 0.4) (layer F.Cu) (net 2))
 (segment (start 153.5 71.3) (end 154.35 71.3) (width 0.4) (layer F.Cu) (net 2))
 (segment (start 154.95 70.7) (end 157.8 70.7) (width 0.4) (layer F.Cu) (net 2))
 (segment (start 162.450002 68.12) (end 161.170002 69.4) (width 0.4) (layer F.Cu) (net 3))
 (segment (start 163.4 68.12) (end 162.450002 68.12) (width 0.4) (layer F.Cu) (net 3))
 (segment (start 161.170002 69.4) (end 159.5 69.4) (width 0.4) (layer F.Cu) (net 3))
 (segment (start 168.88 68.12) (end 169 68) (width 0.7) (layer F.Cu) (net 3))
 (segment (start 163.4 68.12) (end 168.88 68.12) (width 0.7) (layer F.Cu) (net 3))
 (segment (start 159.5 69.4) (end 159.1 69.4) (width 0.4) (layer F.Cu) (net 3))
 (segment (start 159.1 69.4) (end 157.8 68.1) (width 0.4) (layer F.Cu) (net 3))
 (segment (start 154.35 67.7) (end 154.75 68.1) (width 0.4) (layer F.Cu) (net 3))
 (segment (start 153.5 67.7) (end 154.35 67.7) (width 0.4) (layer F.Cu) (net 3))
 (segment (start 154.75 68.1) (end 157.7 68.1) (width 0.4) (layer F.Cu) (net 3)))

